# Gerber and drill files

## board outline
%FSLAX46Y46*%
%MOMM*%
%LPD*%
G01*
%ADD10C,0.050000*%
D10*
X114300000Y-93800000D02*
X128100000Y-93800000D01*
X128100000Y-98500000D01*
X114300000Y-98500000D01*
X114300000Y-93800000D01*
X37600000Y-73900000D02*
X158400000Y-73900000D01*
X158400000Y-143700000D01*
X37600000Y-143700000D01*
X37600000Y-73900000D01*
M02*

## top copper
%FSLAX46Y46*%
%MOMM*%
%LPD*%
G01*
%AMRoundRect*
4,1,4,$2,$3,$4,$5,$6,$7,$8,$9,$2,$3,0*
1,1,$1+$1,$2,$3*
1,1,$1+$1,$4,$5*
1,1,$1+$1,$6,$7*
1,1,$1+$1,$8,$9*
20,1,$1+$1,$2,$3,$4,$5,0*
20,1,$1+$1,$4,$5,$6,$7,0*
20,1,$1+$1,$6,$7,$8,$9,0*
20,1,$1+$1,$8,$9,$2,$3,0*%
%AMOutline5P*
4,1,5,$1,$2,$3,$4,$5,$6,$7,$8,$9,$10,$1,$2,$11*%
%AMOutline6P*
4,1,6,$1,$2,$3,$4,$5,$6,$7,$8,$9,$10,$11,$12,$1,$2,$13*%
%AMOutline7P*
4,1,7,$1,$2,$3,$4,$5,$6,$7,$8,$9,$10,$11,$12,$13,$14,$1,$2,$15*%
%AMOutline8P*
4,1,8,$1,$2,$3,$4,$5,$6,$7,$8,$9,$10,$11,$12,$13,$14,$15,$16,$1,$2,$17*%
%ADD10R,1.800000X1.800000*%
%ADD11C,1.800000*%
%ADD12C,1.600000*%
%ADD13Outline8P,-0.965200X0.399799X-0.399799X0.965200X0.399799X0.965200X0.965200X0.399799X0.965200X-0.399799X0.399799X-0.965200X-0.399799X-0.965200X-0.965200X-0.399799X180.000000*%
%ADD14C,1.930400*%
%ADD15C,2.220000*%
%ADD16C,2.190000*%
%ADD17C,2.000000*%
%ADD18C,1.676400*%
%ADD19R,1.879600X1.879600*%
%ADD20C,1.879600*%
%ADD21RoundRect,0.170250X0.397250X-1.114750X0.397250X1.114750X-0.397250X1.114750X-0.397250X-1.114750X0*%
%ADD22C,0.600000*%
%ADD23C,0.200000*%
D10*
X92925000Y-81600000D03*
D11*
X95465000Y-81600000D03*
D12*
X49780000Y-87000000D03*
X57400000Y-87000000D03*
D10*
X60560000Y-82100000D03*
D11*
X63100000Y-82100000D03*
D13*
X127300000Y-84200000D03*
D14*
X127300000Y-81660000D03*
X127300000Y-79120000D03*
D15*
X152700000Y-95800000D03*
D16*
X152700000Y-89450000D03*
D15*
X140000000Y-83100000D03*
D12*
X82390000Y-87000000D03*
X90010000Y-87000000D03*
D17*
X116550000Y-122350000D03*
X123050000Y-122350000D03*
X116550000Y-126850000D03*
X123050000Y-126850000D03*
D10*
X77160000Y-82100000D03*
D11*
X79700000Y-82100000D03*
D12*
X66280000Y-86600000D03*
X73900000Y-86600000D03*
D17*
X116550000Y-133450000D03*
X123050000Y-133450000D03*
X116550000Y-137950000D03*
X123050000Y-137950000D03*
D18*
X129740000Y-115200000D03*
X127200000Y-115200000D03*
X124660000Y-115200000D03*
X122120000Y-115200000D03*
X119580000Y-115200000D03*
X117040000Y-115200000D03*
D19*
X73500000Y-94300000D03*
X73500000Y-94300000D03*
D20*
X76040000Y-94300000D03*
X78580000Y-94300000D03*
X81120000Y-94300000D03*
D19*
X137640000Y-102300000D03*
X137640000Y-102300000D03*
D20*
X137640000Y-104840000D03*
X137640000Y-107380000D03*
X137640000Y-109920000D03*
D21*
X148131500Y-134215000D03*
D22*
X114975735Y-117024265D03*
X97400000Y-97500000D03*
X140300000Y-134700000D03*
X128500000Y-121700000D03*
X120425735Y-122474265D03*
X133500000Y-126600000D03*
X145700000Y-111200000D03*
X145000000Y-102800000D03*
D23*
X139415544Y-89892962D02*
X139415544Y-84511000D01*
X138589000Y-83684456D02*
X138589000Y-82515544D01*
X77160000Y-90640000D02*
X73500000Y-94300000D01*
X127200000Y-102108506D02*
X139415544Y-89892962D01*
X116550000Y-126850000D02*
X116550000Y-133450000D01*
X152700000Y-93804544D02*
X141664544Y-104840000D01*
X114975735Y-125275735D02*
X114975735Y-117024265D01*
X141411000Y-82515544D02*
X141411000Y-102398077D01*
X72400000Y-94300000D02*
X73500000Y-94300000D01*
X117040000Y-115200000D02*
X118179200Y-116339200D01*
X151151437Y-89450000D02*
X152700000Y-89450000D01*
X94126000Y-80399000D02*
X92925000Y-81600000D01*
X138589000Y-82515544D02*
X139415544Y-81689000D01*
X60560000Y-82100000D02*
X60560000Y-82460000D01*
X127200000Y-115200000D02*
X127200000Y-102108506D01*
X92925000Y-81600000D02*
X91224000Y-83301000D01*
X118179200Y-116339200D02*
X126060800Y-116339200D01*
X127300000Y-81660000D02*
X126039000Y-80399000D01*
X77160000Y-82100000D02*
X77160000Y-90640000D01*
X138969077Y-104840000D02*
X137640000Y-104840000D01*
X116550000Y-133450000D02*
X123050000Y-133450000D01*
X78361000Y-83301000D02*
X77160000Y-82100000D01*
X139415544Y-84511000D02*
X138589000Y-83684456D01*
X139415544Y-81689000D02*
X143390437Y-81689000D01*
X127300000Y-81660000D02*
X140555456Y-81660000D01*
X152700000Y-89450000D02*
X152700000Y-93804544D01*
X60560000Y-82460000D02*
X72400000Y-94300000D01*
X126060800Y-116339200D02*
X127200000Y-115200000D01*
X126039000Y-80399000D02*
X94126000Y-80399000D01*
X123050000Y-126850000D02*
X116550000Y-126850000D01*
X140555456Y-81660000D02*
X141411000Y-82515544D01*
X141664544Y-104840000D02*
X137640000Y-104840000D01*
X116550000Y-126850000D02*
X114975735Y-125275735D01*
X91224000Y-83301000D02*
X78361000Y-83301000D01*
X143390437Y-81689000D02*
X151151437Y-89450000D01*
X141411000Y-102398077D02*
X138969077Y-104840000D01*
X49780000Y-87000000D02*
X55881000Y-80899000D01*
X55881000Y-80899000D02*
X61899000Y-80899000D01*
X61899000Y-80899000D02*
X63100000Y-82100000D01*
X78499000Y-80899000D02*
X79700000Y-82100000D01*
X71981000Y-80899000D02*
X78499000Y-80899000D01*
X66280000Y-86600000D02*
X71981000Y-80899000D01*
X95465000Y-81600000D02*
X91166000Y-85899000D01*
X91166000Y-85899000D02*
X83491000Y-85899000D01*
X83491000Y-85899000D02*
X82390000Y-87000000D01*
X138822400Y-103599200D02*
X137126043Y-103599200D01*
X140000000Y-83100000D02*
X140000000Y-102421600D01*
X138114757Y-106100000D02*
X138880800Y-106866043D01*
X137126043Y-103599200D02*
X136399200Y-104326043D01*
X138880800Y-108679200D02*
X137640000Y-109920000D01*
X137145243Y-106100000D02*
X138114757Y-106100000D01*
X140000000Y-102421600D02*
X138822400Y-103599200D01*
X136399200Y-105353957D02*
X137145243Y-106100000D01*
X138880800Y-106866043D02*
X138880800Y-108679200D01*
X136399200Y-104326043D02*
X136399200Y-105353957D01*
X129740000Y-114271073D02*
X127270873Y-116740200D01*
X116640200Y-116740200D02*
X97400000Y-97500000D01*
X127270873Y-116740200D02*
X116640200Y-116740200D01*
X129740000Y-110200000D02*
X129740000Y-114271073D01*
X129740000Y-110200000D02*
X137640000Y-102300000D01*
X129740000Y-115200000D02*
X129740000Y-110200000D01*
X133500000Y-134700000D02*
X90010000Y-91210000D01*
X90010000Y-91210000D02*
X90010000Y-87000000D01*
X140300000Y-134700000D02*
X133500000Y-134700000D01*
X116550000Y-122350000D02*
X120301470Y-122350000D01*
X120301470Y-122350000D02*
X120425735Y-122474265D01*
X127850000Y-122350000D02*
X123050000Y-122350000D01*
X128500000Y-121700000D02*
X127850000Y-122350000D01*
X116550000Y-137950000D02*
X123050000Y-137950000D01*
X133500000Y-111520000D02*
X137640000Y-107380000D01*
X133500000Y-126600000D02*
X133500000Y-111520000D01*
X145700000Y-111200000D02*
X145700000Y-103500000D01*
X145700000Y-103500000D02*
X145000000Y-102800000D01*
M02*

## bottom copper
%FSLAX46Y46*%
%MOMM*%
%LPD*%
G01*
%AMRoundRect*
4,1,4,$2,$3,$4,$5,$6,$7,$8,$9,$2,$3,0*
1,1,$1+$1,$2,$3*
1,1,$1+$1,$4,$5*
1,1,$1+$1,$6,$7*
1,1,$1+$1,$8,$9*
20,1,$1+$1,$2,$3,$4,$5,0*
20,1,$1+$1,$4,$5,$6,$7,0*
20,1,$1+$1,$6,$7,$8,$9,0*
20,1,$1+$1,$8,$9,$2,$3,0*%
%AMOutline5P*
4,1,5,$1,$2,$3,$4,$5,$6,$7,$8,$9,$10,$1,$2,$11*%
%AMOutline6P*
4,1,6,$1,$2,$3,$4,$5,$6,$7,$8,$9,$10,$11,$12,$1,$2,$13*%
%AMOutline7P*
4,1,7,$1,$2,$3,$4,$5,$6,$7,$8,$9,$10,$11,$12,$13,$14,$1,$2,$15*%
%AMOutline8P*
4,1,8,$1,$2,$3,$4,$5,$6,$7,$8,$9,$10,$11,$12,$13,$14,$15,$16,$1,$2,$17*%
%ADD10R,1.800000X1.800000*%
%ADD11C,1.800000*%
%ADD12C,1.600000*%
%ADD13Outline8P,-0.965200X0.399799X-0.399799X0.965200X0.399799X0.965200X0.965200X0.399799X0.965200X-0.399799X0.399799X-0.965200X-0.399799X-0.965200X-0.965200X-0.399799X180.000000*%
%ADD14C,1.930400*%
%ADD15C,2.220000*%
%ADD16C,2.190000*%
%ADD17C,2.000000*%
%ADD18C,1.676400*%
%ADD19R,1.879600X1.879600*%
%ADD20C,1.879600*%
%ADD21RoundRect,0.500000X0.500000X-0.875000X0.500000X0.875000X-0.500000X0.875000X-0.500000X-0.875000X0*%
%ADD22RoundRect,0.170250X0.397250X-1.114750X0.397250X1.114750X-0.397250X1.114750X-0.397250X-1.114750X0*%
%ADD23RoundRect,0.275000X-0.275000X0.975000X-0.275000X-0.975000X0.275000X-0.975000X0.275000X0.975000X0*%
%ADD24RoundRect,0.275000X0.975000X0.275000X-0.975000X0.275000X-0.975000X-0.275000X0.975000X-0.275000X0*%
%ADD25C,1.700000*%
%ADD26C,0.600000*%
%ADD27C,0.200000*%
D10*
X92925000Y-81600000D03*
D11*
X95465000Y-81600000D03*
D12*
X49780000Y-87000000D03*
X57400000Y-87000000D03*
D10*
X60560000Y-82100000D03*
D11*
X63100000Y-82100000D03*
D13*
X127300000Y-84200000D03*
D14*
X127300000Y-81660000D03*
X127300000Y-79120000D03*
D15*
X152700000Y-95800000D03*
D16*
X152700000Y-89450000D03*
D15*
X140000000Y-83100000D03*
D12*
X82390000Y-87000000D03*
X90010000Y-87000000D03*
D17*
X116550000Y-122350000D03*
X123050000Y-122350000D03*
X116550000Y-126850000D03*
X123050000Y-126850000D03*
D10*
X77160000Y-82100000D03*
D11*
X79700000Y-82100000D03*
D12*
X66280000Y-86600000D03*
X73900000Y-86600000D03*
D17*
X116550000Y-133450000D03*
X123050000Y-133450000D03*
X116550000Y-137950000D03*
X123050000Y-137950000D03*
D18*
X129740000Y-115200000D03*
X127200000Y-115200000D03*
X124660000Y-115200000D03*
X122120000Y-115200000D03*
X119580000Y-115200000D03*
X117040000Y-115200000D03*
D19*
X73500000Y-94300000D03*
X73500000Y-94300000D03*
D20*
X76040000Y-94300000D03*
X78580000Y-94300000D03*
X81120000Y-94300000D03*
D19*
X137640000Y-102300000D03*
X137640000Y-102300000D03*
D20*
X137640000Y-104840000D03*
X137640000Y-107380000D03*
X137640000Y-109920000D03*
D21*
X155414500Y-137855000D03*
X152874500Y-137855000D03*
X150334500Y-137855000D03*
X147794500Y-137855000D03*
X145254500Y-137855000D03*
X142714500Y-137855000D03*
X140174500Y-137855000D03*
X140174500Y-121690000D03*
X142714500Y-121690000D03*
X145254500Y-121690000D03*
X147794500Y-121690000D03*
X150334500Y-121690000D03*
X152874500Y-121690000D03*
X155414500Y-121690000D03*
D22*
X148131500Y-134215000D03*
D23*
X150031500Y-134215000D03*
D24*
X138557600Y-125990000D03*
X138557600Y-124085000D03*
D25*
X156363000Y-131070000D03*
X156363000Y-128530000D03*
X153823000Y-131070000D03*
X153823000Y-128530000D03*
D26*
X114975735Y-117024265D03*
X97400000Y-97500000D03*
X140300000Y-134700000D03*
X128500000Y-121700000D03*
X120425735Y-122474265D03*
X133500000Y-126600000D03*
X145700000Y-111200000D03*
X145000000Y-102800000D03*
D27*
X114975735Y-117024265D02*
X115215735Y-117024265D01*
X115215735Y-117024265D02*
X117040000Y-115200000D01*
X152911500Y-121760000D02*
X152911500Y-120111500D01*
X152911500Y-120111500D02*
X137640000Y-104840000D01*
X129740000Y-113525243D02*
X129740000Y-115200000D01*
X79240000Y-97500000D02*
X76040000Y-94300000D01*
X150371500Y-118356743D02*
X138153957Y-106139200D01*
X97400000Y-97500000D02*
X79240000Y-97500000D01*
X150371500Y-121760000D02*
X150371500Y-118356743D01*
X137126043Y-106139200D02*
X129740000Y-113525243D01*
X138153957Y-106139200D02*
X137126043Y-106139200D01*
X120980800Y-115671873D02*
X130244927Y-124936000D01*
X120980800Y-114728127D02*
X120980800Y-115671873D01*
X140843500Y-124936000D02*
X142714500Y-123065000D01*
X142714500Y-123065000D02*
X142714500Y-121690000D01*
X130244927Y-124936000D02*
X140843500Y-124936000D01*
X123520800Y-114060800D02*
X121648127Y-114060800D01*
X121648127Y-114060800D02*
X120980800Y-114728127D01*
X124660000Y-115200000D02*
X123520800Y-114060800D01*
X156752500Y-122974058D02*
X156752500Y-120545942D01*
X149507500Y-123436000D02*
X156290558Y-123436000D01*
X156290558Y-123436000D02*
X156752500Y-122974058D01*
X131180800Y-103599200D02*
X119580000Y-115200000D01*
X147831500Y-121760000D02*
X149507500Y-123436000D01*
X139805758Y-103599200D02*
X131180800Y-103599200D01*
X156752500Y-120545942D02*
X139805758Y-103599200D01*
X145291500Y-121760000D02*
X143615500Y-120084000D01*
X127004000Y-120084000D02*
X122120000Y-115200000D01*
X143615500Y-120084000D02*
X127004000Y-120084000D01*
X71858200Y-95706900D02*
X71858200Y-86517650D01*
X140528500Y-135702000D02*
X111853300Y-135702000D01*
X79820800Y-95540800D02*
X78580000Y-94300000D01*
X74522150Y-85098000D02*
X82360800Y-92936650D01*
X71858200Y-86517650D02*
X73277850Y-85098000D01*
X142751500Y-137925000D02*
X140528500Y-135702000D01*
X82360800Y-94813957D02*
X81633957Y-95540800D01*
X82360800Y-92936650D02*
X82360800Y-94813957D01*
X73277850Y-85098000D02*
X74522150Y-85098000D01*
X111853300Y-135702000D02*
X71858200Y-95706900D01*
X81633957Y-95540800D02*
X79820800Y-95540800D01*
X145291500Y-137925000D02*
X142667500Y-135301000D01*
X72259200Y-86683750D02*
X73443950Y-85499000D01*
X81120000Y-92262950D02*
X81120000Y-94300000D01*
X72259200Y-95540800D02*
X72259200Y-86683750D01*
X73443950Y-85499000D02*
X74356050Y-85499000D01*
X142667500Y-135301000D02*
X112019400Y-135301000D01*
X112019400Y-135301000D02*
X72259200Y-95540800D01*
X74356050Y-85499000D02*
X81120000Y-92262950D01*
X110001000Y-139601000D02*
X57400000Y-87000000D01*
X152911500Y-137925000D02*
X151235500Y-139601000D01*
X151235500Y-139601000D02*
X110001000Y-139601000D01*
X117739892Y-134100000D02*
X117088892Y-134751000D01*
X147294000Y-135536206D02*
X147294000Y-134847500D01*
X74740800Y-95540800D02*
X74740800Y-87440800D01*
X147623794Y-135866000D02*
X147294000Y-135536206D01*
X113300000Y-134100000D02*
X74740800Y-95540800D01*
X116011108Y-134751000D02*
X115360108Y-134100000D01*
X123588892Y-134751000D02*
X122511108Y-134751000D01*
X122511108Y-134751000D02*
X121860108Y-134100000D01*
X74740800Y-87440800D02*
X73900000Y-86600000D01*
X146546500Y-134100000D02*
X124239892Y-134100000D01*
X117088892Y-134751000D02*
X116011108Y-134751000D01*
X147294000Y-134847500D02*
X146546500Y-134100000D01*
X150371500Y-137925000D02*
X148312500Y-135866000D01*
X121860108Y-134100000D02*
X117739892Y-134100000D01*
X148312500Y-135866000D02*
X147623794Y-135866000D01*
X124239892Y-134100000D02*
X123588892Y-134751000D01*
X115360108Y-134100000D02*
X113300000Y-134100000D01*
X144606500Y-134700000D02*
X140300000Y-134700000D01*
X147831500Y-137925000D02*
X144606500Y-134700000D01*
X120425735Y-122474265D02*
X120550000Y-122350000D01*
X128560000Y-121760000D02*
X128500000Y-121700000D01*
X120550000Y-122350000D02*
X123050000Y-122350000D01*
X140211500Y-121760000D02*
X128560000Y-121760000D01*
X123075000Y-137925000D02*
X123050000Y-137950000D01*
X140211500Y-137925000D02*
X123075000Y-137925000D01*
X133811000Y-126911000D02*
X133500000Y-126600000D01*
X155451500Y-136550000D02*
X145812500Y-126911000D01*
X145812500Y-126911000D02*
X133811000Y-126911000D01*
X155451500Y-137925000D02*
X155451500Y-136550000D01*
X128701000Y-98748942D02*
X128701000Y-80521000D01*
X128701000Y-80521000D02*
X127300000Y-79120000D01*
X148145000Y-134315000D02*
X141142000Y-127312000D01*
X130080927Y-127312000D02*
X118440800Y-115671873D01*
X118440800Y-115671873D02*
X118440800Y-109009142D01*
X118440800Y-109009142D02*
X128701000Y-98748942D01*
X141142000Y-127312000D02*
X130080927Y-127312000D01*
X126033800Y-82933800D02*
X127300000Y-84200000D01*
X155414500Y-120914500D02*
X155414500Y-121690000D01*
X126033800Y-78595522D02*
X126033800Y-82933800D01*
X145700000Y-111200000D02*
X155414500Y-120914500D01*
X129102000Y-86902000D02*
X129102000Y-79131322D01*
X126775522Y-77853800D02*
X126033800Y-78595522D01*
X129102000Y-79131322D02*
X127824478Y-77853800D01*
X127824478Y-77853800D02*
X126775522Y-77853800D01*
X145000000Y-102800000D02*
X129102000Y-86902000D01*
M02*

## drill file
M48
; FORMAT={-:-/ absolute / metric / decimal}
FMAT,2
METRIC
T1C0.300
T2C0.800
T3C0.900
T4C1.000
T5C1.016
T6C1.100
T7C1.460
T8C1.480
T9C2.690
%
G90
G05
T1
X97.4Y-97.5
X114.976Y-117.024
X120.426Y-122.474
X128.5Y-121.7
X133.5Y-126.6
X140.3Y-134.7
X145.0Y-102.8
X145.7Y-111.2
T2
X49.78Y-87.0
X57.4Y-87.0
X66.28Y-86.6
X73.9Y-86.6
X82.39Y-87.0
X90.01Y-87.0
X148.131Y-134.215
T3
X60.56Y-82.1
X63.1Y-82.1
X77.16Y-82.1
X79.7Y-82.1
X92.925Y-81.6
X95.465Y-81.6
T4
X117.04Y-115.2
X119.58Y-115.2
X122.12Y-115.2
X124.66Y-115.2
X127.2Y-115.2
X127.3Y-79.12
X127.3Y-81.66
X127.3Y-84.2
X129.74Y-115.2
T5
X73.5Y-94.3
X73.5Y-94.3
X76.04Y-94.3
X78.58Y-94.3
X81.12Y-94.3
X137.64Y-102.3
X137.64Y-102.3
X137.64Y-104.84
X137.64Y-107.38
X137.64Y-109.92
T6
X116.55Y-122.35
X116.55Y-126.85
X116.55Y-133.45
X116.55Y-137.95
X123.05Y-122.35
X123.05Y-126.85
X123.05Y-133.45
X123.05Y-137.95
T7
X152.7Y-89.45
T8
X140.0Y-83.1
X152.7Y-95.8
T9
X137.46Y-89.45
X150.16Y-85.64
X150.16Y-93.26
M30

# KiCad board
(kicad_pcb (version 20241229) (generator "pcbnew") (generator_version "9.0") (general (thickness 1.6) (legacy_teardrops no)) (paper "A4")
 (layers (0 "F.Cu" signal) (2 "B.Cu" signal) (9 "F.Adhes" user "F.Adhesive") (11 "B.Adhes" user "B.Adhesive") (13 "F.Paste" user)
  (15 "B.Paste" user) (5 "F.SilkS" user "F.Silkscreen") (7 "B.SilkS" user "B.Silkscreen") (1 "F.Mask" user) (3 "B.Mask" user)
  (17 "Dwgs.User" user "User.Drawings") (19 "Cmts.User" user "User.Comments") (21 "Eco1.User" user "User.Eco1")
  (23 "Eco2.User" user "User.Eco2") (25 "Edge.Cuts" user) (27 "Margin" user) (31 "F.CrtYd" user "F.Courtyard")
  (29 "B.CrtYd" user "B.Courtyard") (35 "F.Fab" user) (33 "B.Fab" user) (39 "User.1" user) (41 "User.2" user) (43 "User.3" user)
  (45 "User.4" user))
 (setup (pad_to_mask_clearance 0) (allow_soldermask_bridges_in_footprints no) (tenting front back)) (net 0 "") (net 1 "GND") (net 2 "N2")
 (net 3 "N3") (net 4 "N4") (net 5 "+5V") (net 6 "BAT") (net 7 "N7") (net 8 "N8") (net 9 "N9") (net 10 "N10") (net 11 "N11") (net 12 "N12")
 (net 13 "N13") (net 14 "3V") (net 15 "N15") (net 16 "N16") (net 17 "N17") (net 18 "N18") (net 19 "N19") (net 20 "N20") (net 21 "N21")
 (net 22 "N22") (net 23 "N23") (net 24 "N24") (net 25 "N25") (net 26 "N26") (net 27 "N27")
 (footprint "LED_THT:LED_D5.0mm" (layer "F.Cu") (at 92.925 81.6)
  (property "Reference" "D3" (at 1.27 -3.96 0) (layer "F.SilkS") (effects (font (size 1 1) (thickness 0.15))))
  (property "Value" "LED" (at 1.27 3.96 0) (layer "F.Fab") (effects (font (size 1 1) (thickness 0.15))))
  (pad "1" thru_hole rect (at 0 0) (size 1.8 1.8) (drill 0.9) (layers "*.Cu" "*.Mask") (remove_unused_layers no) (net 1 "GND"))
  (pad "2" thru_hole circle (at 2.54 0) (size 1.8 1.8) (drill 0.9) (layers "*.Cu" "*.Mask") (remove_unused_layers no) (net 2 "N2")))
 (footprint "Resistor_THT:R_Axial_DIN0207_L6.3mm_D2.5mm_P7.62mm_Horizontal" (layer "F.Cu") (at 49.78 87)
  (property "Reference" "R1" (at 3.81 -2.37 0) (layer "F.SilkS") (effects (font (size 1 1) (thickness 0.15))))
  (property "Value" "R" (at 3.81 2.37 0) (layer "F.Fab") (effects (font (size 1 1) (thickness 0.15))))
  (pad "1" thru_hole circle (at 0 0) (size 1.6 1.6) (drill 0.8) (layers "*.Cu" "*.Mask") (remove_unused_layers no) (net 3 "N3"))
  (pad "2" thru_hole circle (at 7.62 0) (size 1.6 1.6) (drill 0.8) (layers "*.Cu" "*.Mask") (remove_unused_layers no) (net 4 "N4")))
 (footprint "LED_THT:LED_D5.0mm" (layer "F.Cu") (at 60.56 82.1)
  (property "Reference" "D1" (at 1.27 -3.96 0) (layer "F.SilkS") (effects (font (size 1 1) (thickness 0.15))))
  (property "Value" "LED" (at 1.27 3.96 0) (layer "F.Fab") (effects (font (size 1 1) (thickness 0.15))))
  (pad "1" thru_hole rect (at 0 0) (size 1.8 1.8) (drill 0.9) (layers "*.Cu" "*.Mask") (remove_unused_layers no) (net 1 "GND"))
  (pad "2" thru_hole circle (at 2.54 0) (size 1.8 1.8) (drill 0.9) (layers "*.Cu" "*.Mask") (remove_unused_layers no) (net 3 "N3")))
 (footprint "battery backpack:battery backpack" (layer "F.Cu") (at 120.45 84.59 -90)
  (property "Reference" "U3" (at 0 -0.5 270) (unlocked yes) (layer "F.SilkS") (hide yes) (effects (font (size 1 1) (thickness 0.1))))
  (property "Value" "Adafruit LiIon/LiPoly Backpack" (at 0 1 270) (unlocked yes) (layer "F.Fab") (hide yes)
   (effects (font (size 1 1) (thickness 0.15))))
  (pad "1" thru_hole roundrect (at -0.39 -6.85 180) (size 1.9304 1.9304) (drill 1) (layers "*.Cu" "*.Mask") (remove_unused_layers no)
   (roundrect_rratio 0.25) (chamfer_ratio 0.2928932188) (chamfer top_left top_right bottom_left bottom_right) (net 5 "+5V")
   (solder_mask_margin 0.0508) (thermal_bridge_angle 0))
  (pad "2" thru_hole circle (at -2.93 -6.85 180) (size 1.9304 1.9304) (drill 1) (layers "*.Cu" "*.Mask") (remove_unused_layers no)
   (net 1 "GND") (solder_mask_margin 0.0508) (thermal_bridge_angle 0))
  (pad "3" thru_hole circle (at -5.47 -6.85 180) (size 1.9304 1.9304) (drill 1) (layers "*.Cu" "*.Mask") (remove_unused_layers no)
   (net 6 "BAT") (solder_mask_margin 0.0508) (thermal_bridge_angle 0)))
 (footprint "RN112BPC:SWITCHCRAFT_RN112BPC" (layer "F.Cu") (at 152.7 89.45)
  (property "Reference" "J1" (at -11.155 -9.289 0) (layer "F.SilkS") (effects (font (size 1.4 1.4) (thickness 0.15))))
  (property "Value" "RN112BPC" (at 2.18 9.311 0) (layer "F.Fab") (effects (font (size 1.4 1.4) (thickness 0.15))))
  (pad "" np_thru_hole circle (at -15.24 0) (size 2.69 2.69) (drill 2.69) (layers "*.Cu" "*.Mask"))
  (pad "" np_thru_hole circle (at -2.54 -3.81) (size 2.69 2.69) (drill 2.69) (layers "*.Cu" "*.Mask"))
  (pad "" np_thru_hole circle (at -2.54 3.81) (size 2.69 2.69) (drill 2.69) (layers "*.Cu" "*.Mask"))
  (pad "R" thru_hole circle (at 0 6.35) (size 2.22 2.22) (drill 1.48) (layers "*.Cu" "*.Mask") (remove_unused_layers no) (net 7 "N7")
   (solder_mask_margin 0.102))
  (pad "S" thru_hole circle (at 0 0) (size 2.19 2.19) (drill 1.46) (layers "*.Cu" "*.Mask") (remove_unused_layers no) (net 1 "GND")
   (solder_mask_margin 0.102))
  (pad "T" thru_hole circle (at -12.7 -6.35) (size 2.22 2.22) (drill 1.48) (layers "*.Cu" "*.Mask") (remove_unused_layers no) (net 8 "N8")
   (solder_mask_margin 0.102)))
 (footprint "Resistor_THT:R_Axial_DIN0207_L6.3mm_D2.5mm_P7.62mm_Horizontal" (layer "F.Cu") (at 82.39 87)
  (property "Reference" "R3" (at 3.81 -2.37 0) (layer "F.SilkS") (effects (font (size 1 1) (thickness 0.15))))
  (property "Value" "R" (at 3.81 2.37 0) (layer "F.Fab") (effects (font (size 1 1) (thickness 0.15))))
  (pad "1" thru_hole circle (at 0 0) (size 1.6 1.6) (drill 0.8) (layers "*.Cu" "*.Mask") (remove_unused_layers no) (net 2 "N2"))
  (pad "2" thru_hole circle (at 7.62 0) (size 1.6 1.6) (drill 0.8) (layers "*.Cu" "*.Mask") (remove_unused_layers no) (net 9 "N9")))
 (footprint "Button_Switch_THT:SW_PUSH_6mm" (layer "F.Cu") (at 116.55 122.35)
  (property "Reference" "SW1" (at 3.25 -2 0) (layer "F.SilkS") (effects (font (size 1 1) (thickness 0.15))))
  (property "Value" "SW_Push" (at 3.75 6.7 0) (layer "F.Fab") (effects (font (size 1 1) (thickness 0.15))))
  (pad "1" thru_hole circle (at 0 0 90) (size 2 2) (drill 1.1) (layers "*.Cu" "*.Mask") (remove_unused_layers no) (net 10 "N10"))
  (pad "1" thru_hole circle (at 6.5 0 90) (size 2 2) (drill 1.1) (layers "*.Cu" "*.Mask") (remove_unused_layers no) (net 10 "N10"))
  (pad "2" thru_hole circle (at 0 4.5 90) (size 2 2) (drill 1.1) (layers "*.Cu" "*.Mask") (remove_unused_layers no) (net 1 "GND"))
  (pad "2" thru_hole circle (at 6.5 4.5 90) (size 2 2) (drill 1.1) (layers "*.Cu" "*.Mask") (remove_unused_layers no) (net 1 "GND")))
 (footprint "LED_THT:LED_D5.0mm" (layer "F.Cu") (at 77.16 82.1)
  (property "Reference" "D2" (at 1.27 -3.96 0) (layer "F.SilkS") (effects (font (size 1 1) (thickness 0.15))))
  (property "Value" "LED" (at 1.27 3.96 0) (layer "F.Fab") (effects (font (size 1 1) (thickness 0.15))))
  (pad "1" thru_hole rect (at 0 0) (size 1.8 1.8) (drill 0.9) (layers "*.Cu" "*.Mask") (remove_unused_layers no) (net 1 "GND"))
  (pad "2" thru_hole circle (at 2.54 0) (size 1.8 1.8) (drill 0.9) (layers "*.Cu" "*.Mask") (remove_unused_layers no) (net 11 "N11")))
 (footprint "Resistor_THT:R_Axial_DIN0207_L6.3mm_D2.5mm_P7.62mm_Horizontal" (layer "F.Cu") (at 66.28 86.6)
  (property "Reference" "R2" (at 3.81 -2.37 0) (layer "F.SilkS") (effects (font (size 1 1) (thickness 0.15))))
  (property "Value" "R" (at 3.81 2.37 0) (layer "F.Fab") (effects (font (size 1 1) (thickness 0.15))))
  (pad "1" thru_hole circle (at 0 0) (size 1.6 1.6) (drill 0.8) (layers "*.Cu" "*.Mask") (remove_unused_layers no) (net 11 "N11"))
  (pad "2" thru_hole circle (at 7.62 0) (size 1.6 1.6) (drill 0.8) (layers "*.Cu" "*.Mask") (remove_unused_layers no) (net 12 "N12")))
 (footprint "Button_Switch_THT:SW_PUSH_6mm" (layer "F.Cu") (at 116.55 133.45)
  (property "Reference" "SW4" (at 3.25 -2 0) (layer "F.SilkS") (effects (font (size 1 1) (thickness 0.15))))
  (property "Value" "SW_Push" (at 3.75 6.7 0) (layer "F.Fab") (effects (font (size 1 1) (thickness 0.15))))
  (pad "1" thru_hole circle (at 0 0 90) (size 2 2) (drill 1.1) (layers "*.Cu" "*.Mask") (remove_unused_layers no) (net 1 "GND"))
  (pad "1" thru_hole circle (at 6.5 0 90) (size 2 2) (drill 1.1) (layers "*.Cu" "*.Mask") (remove_unused_layers no) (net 1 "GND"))
  (pad "2" thru_hole circle (at 0 4.5 90) (size 2 2) (drill 1.1) (layers "*.Cu" "*.Mask") (remove_unused_layers no) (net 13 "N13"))
  (pad "2" thru_hole circle (at 6.5 4.5 90) (size 2 2) (drill 1.1) (layers "*.Cu" "*.Mask") (remove_unused_layers no) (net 13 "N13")))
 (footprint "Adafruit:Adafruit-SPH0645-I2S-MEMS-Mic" (layer "F.Cu") (at 123.39 111.24)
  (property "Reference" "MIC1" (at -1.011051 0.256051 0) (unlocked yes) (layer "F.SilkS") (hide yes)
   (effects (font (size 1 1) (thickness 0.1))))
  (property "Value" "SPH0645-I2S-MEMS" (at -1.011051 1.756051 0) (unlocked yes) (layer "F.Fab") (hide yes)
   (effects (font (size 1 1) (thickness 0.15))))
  (pad "1" thru_hole circle (at 6.35 3.96 90) (size 1.6764 1.6764) (drill 1) (layers "*.Cu" "*.Mask") (remove_unused_layers no)
   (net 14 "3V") (solder_mask_margin 0.0508) (thermal_bridge_angle 0))
  (pad "2" thru_hole circle (at 3.81 3.96 90) (size 1.6764 1.6764) (drill 1) (layers "*.Cu" "*.Mask") (remove_unused_layers no)
   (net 1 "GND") (solder_mask_margin 0.0508) (thermal_bridge_angle 0))
  (pad "3" thru_hole circle (at 1.27 3.96 90) (size 1.6764 1.6764) (drill 1) (layers "*.Cu" "*.Mask") (remove_unused_layers no)
   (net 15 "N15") (solder_mask_margin 0.0508) (thermal_bridge_angle 0))
  (pad "4" thru_hole circle (at -1.27 3.96 90) (size 1.6764 1.6764) (drill 1) (layers "*.Cu" "*.Mask") (remove_unused_layers no)
   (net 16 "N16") (solder_mask_margin 0.0508) (thermal_bridge_angle 0))
  (pad "5" thru_hole circle (at -3.81 3.96 90) (size 1.6764 1.6764) (drill 1) (layers "*.Cu" "*.Mask") (remove_unused_layers no)
   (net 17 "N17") (solder_mask_margin 0.0508) (thermal_bridge_angle 0))
  (pad "6" thru_hole circle (at -6.35 3.96 90) (size 1.6764 1.6764) (drill 1) (layers "*.Cu" "*.Mask") (remove_unused_layers no)
   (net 1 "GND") (solder_mask_margin 0.0508) (thermal_bridge_angle 0)))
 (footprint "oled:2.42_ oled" (layer "F.Cu") (at 77.3 115.8)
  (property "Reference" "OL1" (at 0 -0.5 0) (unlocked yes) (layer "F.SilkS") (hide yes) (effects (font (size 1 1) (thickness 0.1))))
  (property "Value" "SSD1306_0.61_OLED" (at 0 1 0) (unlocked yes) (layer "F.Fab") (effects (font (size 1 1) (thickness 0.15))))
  (pad "1" thru_hole rect (at -3.8 -21.5 90) (size 1.8796 1.8796) (drill 1.016) (layers "*.Cu" "*.Mask") (remove_unused_layers no)
   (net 1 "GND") (solder_mask_margin 0.1016) (thermal_bridge_angle 0))
  (pad "1" thru_hole rect (at -3.8 -21.5 90) (size 1.8796 1.8796) (drill 1.016) (layers "*.Cu" "*.Mask") (remove_unused_layers no)
   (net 1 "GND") (solder_mask_margin 0.1016) (thermal_bridge_angle 0))
  (pad "2" thru_hole circle (at -1.26 -21.5 90) (size 1.8796 1.8796) (drill 1.016) (layers "*.Cu" "*.Mask") (remove_unused_layers no)
   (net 14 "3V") (solder_mask_margin 0.1016) (thermal_bridge_angle 0))
  (pad "3" thru_hole circle (at 1.28 -21.5 90) (size 1.8796 1.8796) (drill 1.016) (layers "*.Cu" "*.Mask") (remove_unused_layers no)
   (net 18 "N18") (solder_mask_margin 0.1016) (thermal_bridge_angle 0))
  (pad "4" thru_hole circle (at 3.82 -21.5 90) (size 1.8796 1.8796) (drill 1.016) (layers "*.Cu" "*.Mask") (remove_unused_layers no)
   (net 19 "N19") (solder_mask_margin 0.1016) (thermal_bridge_angle 0)))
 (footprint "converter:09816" (layer "B.Cu") (at 130.64 105.8 -90)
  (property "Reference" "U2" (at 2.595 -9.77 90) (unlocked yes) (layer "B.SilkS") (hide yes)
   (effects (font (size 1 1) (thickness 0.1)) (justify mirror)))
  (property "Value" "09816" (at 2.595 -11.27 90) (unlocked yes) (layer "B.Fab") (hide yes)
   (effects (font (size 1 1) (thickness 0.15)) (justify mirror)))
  (pad "1" thru_hole rect (at -3.5 -7 180) (size 1.8796 1.8796) (drill 1.016) (layers "*.Cu" "*.Mask") (remove_unused_layers no)
   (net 14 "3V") (solder_mask_margin 0.1016) (thermal_bridge_angle 0))
  (pad "1" thru_hole rect (at -3.5 -7 180) (size 1.8796 1.8796) (drill 1.016) (layers "*.Cu" "*.Mask") (remove_unused_layers no)
   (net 14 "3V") (solder_mask_margin 0.1016) (thermal_bridge_angle 0))
  (pad "2" thru_hole circle (at -0.96 -7 180) (size 1.8796 1.8796) (drill 1.016) (layers "*.Cu" "*.Mask") (remove_unused_layers no)
   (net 1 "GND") (solder_mask_margin 0.1016) (thermal_bridge_angle 0))
  (pad "3" thru_hole circle (at 1.58 -7 180) (size 1.8796 1.8796) (drill 1.016) (layers "*.Cu" "*.Mask") (remove_unused_layers no)
   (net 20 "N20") (solder_mask_margin 0.1016) (thermal_bridge_angle 0))
  (pad "4" thru_hole circle (at 4.12 -7 180) (size 1.8796 1.8796) (drill 1.016) (layers "*.Cu" "*.Mask") (remove_unused_layers no)
   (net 8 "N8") (solder_mask_margin 0.1016) (thermal_bridge_angle 0)))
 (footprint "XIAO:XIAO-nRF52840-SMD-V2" (layer "B.Cu") (at 147.8315 129.815 90)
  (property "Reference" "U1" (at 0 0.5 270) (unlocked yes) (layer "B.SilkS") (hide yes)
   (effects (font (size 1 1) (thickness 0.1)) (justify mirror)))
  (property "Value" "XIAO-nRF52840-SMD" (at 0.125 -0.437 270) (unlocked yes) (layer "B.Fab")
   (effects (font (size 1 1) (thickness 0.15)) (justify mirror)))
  (pad "1" smd roundrect (at -8.04 7.583 90) (size 2.75 2) (layers "B.Cu" "B.Mask" "B.Paste") (roundrect_rratio 0.25) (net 20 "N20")
   (solder_mask_margin 0.0508) (thermal_bridge_angle 45))
  (pad "2" smd roundrect (at -8.04 5.043 90) (size 2.75 2) (layers "B.Cu" "B.Mask" "B.Paste") (roundrect_rratio 0.25) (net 4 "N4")
   (solder_mask_margin 0.0508) (thermal_bridge_angle 45))
  (pad "3" smd roundrect (at -8.04 2.503 90) (size 2.75 2) (layers "B.Cu" "B.Mask" "B.Paste") (roundrect_rratio 0.25) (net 12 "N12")
   (solder_mask_margin 0.0508) (thermal_bridge_angle 45))
  (pad "4" smd roundrect (at -8.04 -0.037 90) (size 2.75 2) (layers "B.Cu" "B.Mask" "B.Paste") (roundrect_rratio 0.25) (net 9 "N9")
   (solder_mask_margin 0.0508) (thermal_bridge_angle 45))
  (pad "5" smd roundrect (at -8.04 -2.577 90) (size 2.75 2) (layers "B.Cu" "B.Mask" "B.Paste") (roundrect_rratio 0.25) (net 19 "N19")
   (solder_mask_margin 0.0508) (thermal_bridge_angle 45))
  (pad "6" smd roundrect (at -8.04 -5.117 90) (size 2.75 2) (layers "B.Cu" "B.Mask" "B.Paste") (roundrect_rratio 0.25) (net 18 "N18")
   (solder_mask_margin 0.0508) (thermal_bridge_angle 45))
  (pad "7" smd roundrect (at -8.04 -7.657 90) (size 2.75 2) (layers "B.Cu" "B.Mask" "B.Paste") (roundrect_rratio 0.25) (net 13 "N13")
   (solder_mask_margin 0.0508) (thermal_bridge_angle 45))
  (pad "8" smd roundrect (at 8.125 -7.657 90) (size 2.75 2) (layers "B.Cu" "B.Mask" "B.Paste") (roundrect_rratio 0.25) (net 10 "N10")
   (solder_mask_margin 0.0508) (thermal_bridge_angle 45))
  (pad "9" smd roundrect (at 8.125 -5.117 90) (size 2.75 2) (layers "B.Cu" "B.Mask" "B.Paste") (roundrect_rratio 0.25) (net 15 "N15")
   (solder_mask_margin 0.0508) (thermal_bridge_angle 45))
  (pad "10" smd roundrect (at 8.125 -2.577 90) (size 2.75 2) (layers "B.Cu" "B.Mask" "B.Paste") (roundrect_rratio 0.25) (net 16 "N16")
   (solder_mask_margin 0.0508) (thermal_bridge_angle 45))
  (pad "11" smd roundrect (at 8.125 -0.037 90) (size 2.75 2) (layers "B.Cu" "B.Mask" "B.Paste") (roundrect_rratio 0.25) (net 17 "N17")
   (solder_mask_margin 0.0508) (thermal_bridge_angle 45))
  (pad "12" smd roundrect (at 8.125 2.503 90) (size 2.75 2) (layers "B.Cu" "B.Mask" "B.Paste") (roundrect_rratio 0.25) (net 14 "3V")
   (solder_mask_margin 0.0508) (thermal_bridge_angle 45))
  (pad "13" smd roundrect (at 8.125 5.043 90) (size 2.75 2) (layers "B.Cu" "B.Mask" "B.Paste") (roundrect_rratio 0.25) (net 1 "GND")
   (solder_mask_margin 0.0508) (thermal_bridge_angle 45))
  (pad "14" smd roundrect (at 8.125 7.583 90) (size 2.75 2) (layers "B.Cu" "B.Mask" "B.Paste") (roundrect_rratio 0.25) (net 5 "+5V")
   (solder_mask_margin 0.0508) (thermal_bridge_angle 45))
  (pad "15" thru_hole roundrect (at -4.4 0.3 90) (size 2.57 1.135) (drill 0.8) (layers "*.Cu" "*.Mask") (remove_unused_layers no)
   (roundrect_rratio 0.15) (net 6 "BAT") (thermal_bridge_angle 45))
  (pad "16" smd roundrect (at -4.4 2.2 270) (size 2.5 1.1) (layers "B.Cu" "B.Mask" "B.Paste") (roundrect_rratio 0.25) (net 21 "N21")
   (solder_mask_margin 0.0508) (thermal_bridge_angle 45))
  (pad "17" smd roundrect (at 3.825 -9.2739 180) (size 2.5 1.1) (layers "B.Cu" "B.Mask" "B.Paste") (roundrect_rratio 0.25) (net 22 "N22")
   (solder_mask_margin 0.0508) (thermal_bridge_angle 45))
  (pad "18" smd roundrect (at 5.73 -9.2739 180) (size 2.5 1.1) (layers "B.Cu" "B.Mask" "B.Paste") (roundrect_rratio 0.25) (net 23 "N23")
   (solder_mask_margin 0.0508) (thermal_bridge_angle 45))
  (pad "19" smd circle (at -1.255 8.5315 90) (size 1.7 1.7) (layers "B.Cu" "B.Mask" "B.Paste") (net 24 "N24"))
  (pad "20" smd circle (at 1.285 8.5315 90) (size 1.7 1.7) (layers "B.Cu" "B.Mask" "B.Paste") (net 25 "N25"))
  (pad "21" smd circle (at -1.255 5.9915 90) (size 1.7 1.7) (layers "B.Cu" "B.Mask" "B.Paste") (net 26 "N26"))
  (pad "22" smd circle (at 1.285 5.9915 90) (size 1.7 1.7) (layers "B.Cu" "B.Mask" "B.Paste") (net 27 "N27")))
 (gr_rect (start 114.3 93.8) (end 128.1 98.5) (stroke (width 0.05) (type default)) (fill no) (layer "Edge.Cuts"))
 (gr_rect (start 37.6 73.9) (end 158.4 143.7) (stroke (width 0.05) (type default)) (fill no) (layer "Edge.Cuts"))
 (segment (start 139.415544 89.892962) (end 139.415544 84.511) (width 0.2) (layer "F.Cu") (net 1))
 (segment (start 138.589 83.684456) (end 138.589 82.515544) (width 0.2) (layer "F.Cu") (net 1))
 (segment (start 77.16 90.64) (end 73.5 94.3) (width 0.2) (layer "F.Cu") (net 1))
 (segment (start 127.2 102.108506) (end 139.415544 89.892962) (width 0.2) (layer "F.Cu") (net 1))
 (segment (start 116.55 126.85) (end 116.55 133.45) (width 0.2) (layer "F.Cu") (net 1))
 (segment (start 152.7 93.804544) (end 141.664544 104.84) (width 0.2) (layer "F.Cu") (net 1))
 (segment (start 114.975735 125.275735) (end 114.975735 117.024265) (width 0.2) (layer "F.Cu") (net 1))
 (segment (start 141.411 82.515544) (end 141.411 102.398077) (width 0.2) (layer "F.Cu") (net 1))
 (segment (start 72.4 94.3) (end 73.5 94.3) (width 0.2) (layer "F.Cu") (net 1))
 (segment (start 117.04 115.2) (end 118.1792 116.3392) (width 0.2) (layer "F.Cu") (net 1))
 (segment (start 151.151437 89.45) (end 152.7 89.45) (width 0.2) (layer "F.Cu") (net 1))
 (segment (start 94.126 80.399) (end 92.925 81.6) (width 0.2) (layer "F.Cu") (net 1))
 (segment (start 138.589 82.515544) (end 139.415544 81.689) (width 0.2) (layer "F.Cu") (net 1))
 (segment (start 60.56 82.1) (end 60.56 82.46) (width 0.2) (layer "F.Cu") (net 1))
 (segment (start 127.2 115.2) (end 127.2 102.108506) (width 0.2) (layer "F.Cu") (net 1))
 (segment (start 92.925 81.6) (end 91.224 83.301) (width 0.2) (layer "F.Cu") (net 1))
 (segment (start 118.1792 116.3392) (end 126.0608 116.3392) (width 0.2) (layer "F.Cu") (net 1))
 (segment (start 127.3 81.66) (end 126.039 80.399) (width 0.2) (layer "F.Cu") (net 1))
 (segment (start 77.16 82.1) (end 77.16 90.64) (width 0.2) (layer "F.Cu") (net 1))
 (segment (start 138.969077 104.84) (end 137.64 104.84) (width 0.2) (layer "F.Cu") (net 1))
 (segment (start 116.55 133.45) (end 123.05 133.45) (width 0.2) (layer "F.Cu") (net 1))
 (segment (start 78.361 83.301) (end 77.16 82.1) (width 0.2) (layer "F.Cu") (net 1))
 (segment (start 139.415544 84.511) (end 138.589 83.684456) (width 0.2) (layer "F.Cu") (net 1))
 (segment (start 139.415544 81.689) (end 143.390437 81.689) (width 0.2) (layer "F.Cu") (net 1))
 (segment (start 127.3 81.66) (end 140.555456 81.66) (width 0.2) (layer "F.Cu") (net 1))
 (segment (start 152.7 89.45) (end 152.7 93.804544) (width 0.2) (layer "F.Cu") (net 1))
 (segment (start 60.56 82.46) (end 72.4 94.3) (width 0.2) (layer "F.Cu") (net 1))
 (segment (start 126.0608 116.3392) (end 127.2 115.2) (width 0.2) (layer "F.Cu") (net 1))
 (segment (start 126.039 80.399) (end 94.126 80.399) (width 0.2) (layer "F.Cu") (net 1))
 (segment (start 123.05 126.85) (end 116.55 126.85) (width 0.2) (layer "F.Cu") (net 1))
 (segment (start 140.555456 81.66) (end 141.411 82.515544) (width 0.2) (layer "F.Cu") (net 1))
 (segment (start 141.664544 104.84) (end 137.64 104.84) (width 0.2) (layer "F.Cu") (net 1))
 (segment (start 116.55 126.85) (end 114.975735 125.275735) (width 0.2) (layer "F.Cu") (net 1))
 (segment (start 91.224 83.301) (end 78.361 83.301) (width 0.2) (layer "F.Cu") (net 1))
 (segment (start 143.390437 81.689) (end 151.151437 89.45) (width 0.2) (layer "F.Cu") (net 1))
 (segment (start 141.411 102.398077) (end 138.969077 104.84) (width 0.2) (layer "F.Cu") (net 1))
 (via (at 114.975735 117.024265) (size 0.6) (drill 0.3) (layers "F.Cu" "B.Cu") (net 1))
 (segment (start 114.975735 117.024265) (end 115.215735 117.024265) (width 0.2) (layer "B.Cu") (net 1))
 (segment (start 115.215735 117.024265) (end 117.04 115.2) (width 0.2) (layer "B.Cu") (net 1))
 (segment (start 152.9115 121.76) (end 152.9115 120.1115) (width 0.2) (layer "B.Cu") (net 1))
 (segment (start 152.9115 120.1115) (end 137.64 104.84) (width 0.2) (layer "B.Cu") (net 1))
 (segment (start 49.78 87) (end 55.881 80.899) (width 0.2) (layer "F.Cu") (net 3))
 (segment (start 55.881 80.899) (end 61.899 80.899) (width 0.2) (layer "F.Cu") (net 3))
 (segment (start 61.899 80.899) (end 63.1 82.1) (width 0.2) (layer "F.Cu") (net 3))
 (segment (start 78.499 80.899) (end 79.7 82.1) (width 0.2) (layer "F.Cu") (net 11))
 (segment (start 71.981 80.899) (end 78.499 80.899) (width 0.2) (layer "F.Cu") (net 11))
 (segment (start 66.28 86.6) (end 71.981 80.899) (width 0.2) (layer "F.Cu") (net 11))
 (segment (start 95.465 81.6) (end 91.166 85.899) (width 0.2) (layer "F.Cu") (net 2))
 (segment (start 91.166 85.899) (end 83.491 85.899) (width 0.2) (layer "F.Cu") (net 2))
 (segment (start 83.491 85.899) (end 82.39 87) (width 0.2) (layer "F.Cu") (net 2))
 (segment (start 138.8224 103.5992) (end 137.126043 103.5992) (width 0.2) (layer "F.Cu") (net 8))
 (segment (start 140 83.1) (end 140 102.4216) (width 0.2) (layer "F.Cu") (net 8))
 (segment (start 138.114757 106.1) (end 138.8808 106.866043) (width 0.2) (layer "F.Cu") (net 8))
 (segment (start 137.126043 103.5992) (end 136.3992 104.326043) (width 0.2) (layer "F.Cu") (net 8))
 (segment (start 138.8808 108.6792) (end 137.64 109.92) (width 0.2) (layer "F.Cu") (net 8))
 (segment (start 137.145243 106.1) (end 138.114757 106.1) (width 0.2) (layer "F.Cu") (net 8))
 (segment (start 140 102.4216) (end 138.8224 103.5992) (width 0.2) (layer "F.Cu") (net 8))
 (segment (start 136.3992 105.353957) (end 137.145243 106.1) (width 0.2) (layer "F.Cu") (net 8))
 (segment (start 138.8808 106.866043) (end 138.8808 108.6792) (width 0.2) (layer "F.Cu") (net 8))
 (segment (start 136.3992 104.326043) (end 136.3992 105.353957) (width 0.2) (layer "F.Cu") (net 8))
 (segment (start 129.74 114.271073) (end 127.270873 116.7402) (width 0.2) (layer "F.Cu") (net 14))
 (segment (start 116.6402 116.7402) (end 97.4 97.5) (width 0.2) (layer "F.Cu") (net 14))
 (segment (start 127.270873 116.7402) (end 116.6402 116.7402) (width 0.2) (layer "F.Cu") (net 14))
 (segment (start 129.74 110.2) (end 129.74 114.271073) (width 0.2) (layer "F.Cu") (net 14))
 (segment (start 129.74 110.2) (end 137.64 102.3) (width 0.2) (layer "F.Cu") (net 14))
 (segment (start 129.74 115.2) (end 129.74 110.2) (width 0.2) (layer "F.Cu") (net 14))
 (via (at 97.4 97.5) (size 0.6) (drill 0.3) (layers "F.Cu" "B.Cu") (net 14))
 (segment (start 129.74 113.525243) (end 129.74 115.2) (width 0.2) (layer "B.Cu") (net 14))
 (segment (start 79.24 97.5) (end 76.04 94.3) (width 0.2) (layer "B.Cu") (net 14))
 (segment (start 150.3715 118.356743) (end 138.153957 106.1392) (width 0.2) (layer "B.Cu") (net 14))
 (segment (start 97.4 97.5) (end 79.24 97.5) (width 0.2) (layer "B.Cu") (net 14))
 (segment (start 150.3715 121.76) (end 150.3715 118.356743) (width 0.2) (layer "B.Cu") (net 14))
 (segment (start 137.126043 106.1392) (end 129.74 113.525243) (width 0.2) (layer "B.Cu") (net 14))
 (segment (start 138.153957 106.1392) (end 137.126043 106.1392) (width 0.2) (layer "B.Cu") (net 14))
 (segment (start 120.9808 115.671873) (end 130.244927 124.936) (width 0.2) (layer "B.Cu") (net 15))
 (segment (start 120.9808 114.728127) (end 120.9808 115.671873) (width 0.2) (layer "B.Cu") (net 15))
 (segment (start 140.8435 124.936) (end 142.7145 123.065) (width 0.2) (layer "B.Cu") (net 15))
 (segment (start 142.7145 123.065) (end 142.7145 121.69) (width 0.2) (layer "B.Cu") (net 15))
 (segment (start 130.244927 124.936) (end 140.8435 124.936) (width 0.2) (layer "B.Cu") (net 15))
 (segment (start 123.5208 114.0608) (end 121.648127 114.0608) (width 0.2) (layer "B.Cu") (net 15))
 (segment (start 121.648127 114.0608) (end 120.9808 114.728127) (width 0.2) (layer "B.Cu") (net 15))
 (segment (start 124.66 115.2) (end 123.5208 114.0608) (width 0.2) (layer "B.Cu") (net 15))
 (segment (start 156.7525 122.974058) (end 156.7525 120.545942) (width 0.2) (layer "B.Cu") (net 17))
 (segment (start 149.5075 123.436) (end 156.290558 123.436) (width 0.2) (layer "B.Cu") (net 17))
 (segment (start 156.290558 123.436) (end 156.7525 122.974058) (width 0.2) (layer "B.Cu") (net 17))
 (segment (start 131.1808 103.5992) (end 119.58 115.2) (width 0.2) (layer "B.Cu") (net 17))
 (segment (start 147.8315 121.76) (end 149.5075 123.436) (width 0.2) (layer "B.Cu") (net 17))
 (segment (start 139.805758 103.5992) (end 131.1808 103.5992) (width 0.2) (layer "B.Cu") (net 17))
 (segment (start 156.7525 120.545942) (end 139.805758 103.5992) (width 0.2) (layer "B.Cu") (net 17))
 (segment (start 145.2915 121.76) (end 143.6155 120.084) (width 0.2) (layer "B.Cu") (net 16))
 (segment (start 127.004 120.084) (end 122.12 115.2) (width 0.2) (layer "B.Cu") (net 16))
 (segment (start 143.6155 120.084) (end 127.004 120.084) (width 0.2) (layer "B.Cu") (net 16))
 (segment (start 71.8582 95.7069) (end 71.8582 86.51765) (width 0.2) (layer "B.Cu") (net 18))
 (segment (start 140.5285 135.702) (end 111.8533 135.702) (width 0.2) (layer "B.Cu") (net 18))
 (segment (start 79.8208 95.5408) (end 78.58 94.3) (width 0.2) (layer "B.Cu") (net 18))
 (segment (start 74.52215 85.098) (end 82.3608 92.93665) (width 0.2) (layer "B.Cu") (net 18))
 (segment (start 71.8582 86.51765) (end 73.27785 85.098) (width 0.2) (layer "B.Cu") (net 18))
 (segment (start 142.7515 137.925) (end 140.5285 135.702) (width 0.2) (layer "B.Cu") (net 18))
 (segment (start 82.3608 94.813957) (end 81.633957 95.5408) (width 0.2) (layer "B.Cu") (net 18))
 (segment (start 82.3608 92.93665) (end 82.3608 94.813957) (width 0.2) (layer "B.Cu") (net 18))
 (segment (start 73.27785 85.098) (end 74.52215 85.098) (width 0.2) (layer "B.Cu") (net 18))
 (segment (start 111.8533 135.702) (end 71.8582 95.7069) (width 0.2) (layer "B.Cu") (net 18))
 (segment (start 81.633957 95.5408) (end 79.8208 95.5408) (width 0.2) (layer "B.Cu") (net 18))
 (segment (start 145.2915 137.925) (end 142.6675 135.301) (width 0.2) (layer "B.Cu") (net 19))
 (segment (start 72.2592 86.68375) (end 73.44395 85.499) (width 0.2) (layer "B.Cu") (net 19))
 (segment (start 81.12 92.26295) (end 81.12 94.3) (width 0.2) (layer "B.Cu") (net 19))
 (segment (start 72.2592 95.5408) (end 72.2592 86.68375) (width 0.2) (layer "B.Cu") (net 19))
 (segment (start 73.44395 85.499) (end 74.35605 85.499) (width 0.2) (layer "B.Cu") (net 19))
 (segment (start 142.6675 135.301) (end 112.0194 135.301) (width 0.2) (layer "B.Cu") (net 19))
 (segment (start 112.0194 135.301) (end 72.2592 95.5408) (width 0.2) (layer "B.Cu") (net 19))
 (segment (start 74.35605 85.499) (end 81.12 92.26295) (width 0.2) (layer "B.Cu") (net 19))
 (segment (start 110.001 139.601) (end 57.4 87) (width 0.2) (layer "B.Cu") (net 4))
 (segment (start 152.9115 137.925) (end 151.2355 139.601) (width 0.2) (layer "B.Cu") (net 4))
 (segment (start 151.2355 139.601) (end 110.001 139.601) (width 0.2) (layer "B.Cu") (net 4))
 (segment (start 117.739892 134.1) (end 117.088892 134.751) (width 0.2) (layer "B.Cu") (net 12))
 (segment (start 147.294 135.536206) (end 147.294 134.8475) (width 0.2) (layer "B.Cu") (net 12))
 (segment (start 74.7408 95.5408) (end 74.7408 87.4408) (width 0.2) (layer "B.Cu") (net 12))
 (segment (start 147.623794 135.866) (end 147.294 135.536206) (width 0.2) (layer "B.Cu") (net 12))
 (segment (start 113.3 134.1) (end 74.7408 95.5408) (width 0.2) (layer "B.Cu") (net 12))
 (segment (start 116.011108 134.751) (end 115.360108 134.1) (width 0.2) (layer "B.Cu") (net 12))
 (segment (start 123.588892 134.751) (end 122.511108 134.751) (width 0.2) (layer "B.Cu") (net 12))
 (segment (start 122.511108 134.751) (end 121.860108 134.1) (width 0.2) (layer "B.Cu") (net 12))
 (segment (start 74.7408 87.4408) (end 73.9 86.6) (width 0.2) (layer "B.Cu") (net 12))
 (segment (start 146.5465 134.1) (end 124.239892 134.1) (width 0.2) (layer "B.Cu") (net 12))
 (segment (start 117.088892 134.751) (end 116.011108 134.751) (width 0.2) (layer "B.Cu") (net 12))
 (segment (start 147.294 134.8475) (end 146.5465 134.1) (width 0.2) (layer "B.Cu") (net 12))
 (segment (start 150.3715 137.925) (end 148.3125 135.866) (width 0.2) (layer "B.Cu") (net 12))
 (segment (start 121.860108 134.1) (end 117.739892 134.1) (width 0.2) (layer "B.Cu") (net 12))
 (segment (start 148.3125 135.866) (end 147.623794 135.866) (width 0.2) (layer "B.Cu") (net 12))
 (segment (start 124.239892 134.1) (end 123.588892 134.751) (width 0.2) (layer "B.Cu") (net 12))
 (segment (start 115.360108 134.1) (end 113.3 134.1) (width 0.2) (layer "B.Cu") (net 12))
 (segment (start 133.5 134.7) (end 90.01 91.21) (width 0.2) (layer "F.Cu") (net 9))
 (segment (start 90.01 91.21) (end 90.01 87) (width 0.2) (layer "F.Cu") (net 9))
 (segment (start 140.3 134.7) (end 133.5 134.7) (width 0.2) (layer "F.Cu") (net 9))
 (via (at 140.3 134.7) (size 0.6) (drill 0.3) (layers "F.Cu" "B.Cu") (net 9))
 (segment (start 144.6065 134.7) (end 140.3 134.7) (width 0.2) (layer "B.Cu") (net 9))
 (segment (start 147.8315 137.925) (end 144.6065 134.7) (width 0.2) (layer "B.Cu") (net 9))
 (segment (start 116.55 122.35) (end 120.30147 122.35) (width 0.2) (layer "F.Cu") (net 10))
 (segment (start 120.30147 122.35) (end 120.425735 122.474265) (width 0.2) (layer "F.Cu") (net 10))
 (segment (start 127.85 122.35) (end 123.05 122.35) (width 0.2) (layer "F.Cu") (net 10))
 (segment (start 128.5 121.7) (end 127.85 122.35) (width 0.2) (layer "F.Cu") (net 10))
 (via (at 128.5 121.7) (size 0.6) (drill 0.3) (layers "F.Cu" "B.Cu") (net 10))
 (via (at 120.425735 122.474265) (size 0.6) (drill 0.3) (layers "F.Cu" "B.Cu") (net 10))
 (segment (start 120.425735 122.474265) (end 120.55 122.35) (width 0.2) (layer "B.Cu") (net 10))
 (segment (start 128.56 121.76) (end 128.5 121.7) (width 0.2) (layer "B.Cu") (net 10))
 (segment (start 120.55 122.35) (end 123.05 122.35) (width 0.2) (layer "B.Cu") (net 10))
 (segment (start 140.2115 121.76) (end 128.56 121.76) (width 0.2) (layer "B.Cu") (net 10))
 (segment (start 116.55 137.95) (end 123.05 137.95) (width 0.2) (layer "F.Cu") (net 13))
 (segment (start 123.075 137.925) (end 123.05 137.95) (width 0.2) (layer "B.Cu") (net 13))
 (segment (start 140.2115 137.925) (end 123.075 137.925) (width 0.2) (layer "B.Cu") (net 13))
 (segment (start 133.5 111.52) (end 137.64 107.38) (width 0.2) (layer "F.Cu") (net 20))
 (segment (start 133.5 126.6) (end 133.5 111.52) (width 0.2) (layer "F.Cu") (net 20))
 (via (at 133.5 126.6) (size 0.6) (drill 0.3) (layers "F.Cu" "B.Cu") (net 20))
 (segment (start 133.811 126.911) (end 133.5 126.6) (width 0.2) (layer "B.Cu") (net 20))
 (segment (start 155.4515 136.55) (end 145.8125 126.911) (width 0.2) (layer "B.Cu") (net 20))
 (segment (start 145.8125 126.911) (end 133.811 126.911) (width 0.2) (layer "B.Cu") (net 20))
 (segment (start 155.4515 137.925) (end 155.4515 136.55) (width 0.2) (layer "B.Cu") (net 20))
 (segment (start 128.701 98.748942) (end 128.701 80.521) (width 0.2) (layer "B.Cu") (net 6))
 (segment (start 128.701 80.521) (end 127.3 79.12) (width 0.2) (layer "B.Cu") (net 6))
 (segment (start 148.145 134.315) (end 141.142 127.312) (width 0.2) (layer "B.Cu") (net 6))
 (segment (start 130.080927 127.312) (end 118.4408 115.671873) (width 0.2) (layer "B.Cu") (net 6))
 (segment (start 118.4408 115.671873) (end 118.4408 109.009142) (width 0.2) (layer "B.Cu") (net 6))
 (segment (start 118.4408 109.009142) (end 128.701 98.748942) (width 0.2) (layer "B.Cu") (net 6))
 (segment (start 141.142 127.312) (end 130.080927 127.312) (width 0.2) (layer "B.Cu") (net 6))
 (segment (start 145.7 111.2) (end 145.7 103.5) (width 0.2) (layer "F.Cu") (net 5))
 (segment (start 145.7 103.5) (end 145 102.8) (width 0.2) (layer "F.Cu") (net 5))
 (via (at 145.7 111.2) (size 0.6) (drill 0.3) (layers "F.Cu" "B.Cu") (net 5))
 (via (at 145 102.8) (size 0.6) (drill 0.3) (layers "F.Cu" "B.Cu") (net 5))
 (segment (start 126.0338 82.9338) (end 127.3 84.2) (width 0.2) (layer "B.Cu") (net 5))
 (segment (start 155.4145 120.9145) (end 155.4145 121.69) (width 0.2) (layer "B.Cu") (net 5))
 (segment (start 126.0338 78.595522) (end 126.0338 82.9338) (width 0.2) (layer "B.Cu") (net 5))
 (segment (start 145.7 111.2) (end 155.4145 120.9145) (width 0.2) (layer "B.Cu") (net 5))
 (segment (start 129.102 86.902) (end 129.102 79.131322) (width 0.2) (layer "B.Cu") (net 5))
 (segment (start 126.775522 77.8538) (end 126.0338 78.595522) (width 0.2) (layer "B.Cu") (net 5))
 (segment (start 129.102 79.131322) (end 127.824478 77.8538) (width 0.2) (layer "B.Cu") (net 5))
 (segment (start 127.824478 77.8538) (end 126.775522 77.8538) (width 0.2) (layer "B.Cu") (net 5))
 (segment (start 145 102.8) (end 129.102 86.902) (width 0.2) (layer "B.Cu") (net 5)))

